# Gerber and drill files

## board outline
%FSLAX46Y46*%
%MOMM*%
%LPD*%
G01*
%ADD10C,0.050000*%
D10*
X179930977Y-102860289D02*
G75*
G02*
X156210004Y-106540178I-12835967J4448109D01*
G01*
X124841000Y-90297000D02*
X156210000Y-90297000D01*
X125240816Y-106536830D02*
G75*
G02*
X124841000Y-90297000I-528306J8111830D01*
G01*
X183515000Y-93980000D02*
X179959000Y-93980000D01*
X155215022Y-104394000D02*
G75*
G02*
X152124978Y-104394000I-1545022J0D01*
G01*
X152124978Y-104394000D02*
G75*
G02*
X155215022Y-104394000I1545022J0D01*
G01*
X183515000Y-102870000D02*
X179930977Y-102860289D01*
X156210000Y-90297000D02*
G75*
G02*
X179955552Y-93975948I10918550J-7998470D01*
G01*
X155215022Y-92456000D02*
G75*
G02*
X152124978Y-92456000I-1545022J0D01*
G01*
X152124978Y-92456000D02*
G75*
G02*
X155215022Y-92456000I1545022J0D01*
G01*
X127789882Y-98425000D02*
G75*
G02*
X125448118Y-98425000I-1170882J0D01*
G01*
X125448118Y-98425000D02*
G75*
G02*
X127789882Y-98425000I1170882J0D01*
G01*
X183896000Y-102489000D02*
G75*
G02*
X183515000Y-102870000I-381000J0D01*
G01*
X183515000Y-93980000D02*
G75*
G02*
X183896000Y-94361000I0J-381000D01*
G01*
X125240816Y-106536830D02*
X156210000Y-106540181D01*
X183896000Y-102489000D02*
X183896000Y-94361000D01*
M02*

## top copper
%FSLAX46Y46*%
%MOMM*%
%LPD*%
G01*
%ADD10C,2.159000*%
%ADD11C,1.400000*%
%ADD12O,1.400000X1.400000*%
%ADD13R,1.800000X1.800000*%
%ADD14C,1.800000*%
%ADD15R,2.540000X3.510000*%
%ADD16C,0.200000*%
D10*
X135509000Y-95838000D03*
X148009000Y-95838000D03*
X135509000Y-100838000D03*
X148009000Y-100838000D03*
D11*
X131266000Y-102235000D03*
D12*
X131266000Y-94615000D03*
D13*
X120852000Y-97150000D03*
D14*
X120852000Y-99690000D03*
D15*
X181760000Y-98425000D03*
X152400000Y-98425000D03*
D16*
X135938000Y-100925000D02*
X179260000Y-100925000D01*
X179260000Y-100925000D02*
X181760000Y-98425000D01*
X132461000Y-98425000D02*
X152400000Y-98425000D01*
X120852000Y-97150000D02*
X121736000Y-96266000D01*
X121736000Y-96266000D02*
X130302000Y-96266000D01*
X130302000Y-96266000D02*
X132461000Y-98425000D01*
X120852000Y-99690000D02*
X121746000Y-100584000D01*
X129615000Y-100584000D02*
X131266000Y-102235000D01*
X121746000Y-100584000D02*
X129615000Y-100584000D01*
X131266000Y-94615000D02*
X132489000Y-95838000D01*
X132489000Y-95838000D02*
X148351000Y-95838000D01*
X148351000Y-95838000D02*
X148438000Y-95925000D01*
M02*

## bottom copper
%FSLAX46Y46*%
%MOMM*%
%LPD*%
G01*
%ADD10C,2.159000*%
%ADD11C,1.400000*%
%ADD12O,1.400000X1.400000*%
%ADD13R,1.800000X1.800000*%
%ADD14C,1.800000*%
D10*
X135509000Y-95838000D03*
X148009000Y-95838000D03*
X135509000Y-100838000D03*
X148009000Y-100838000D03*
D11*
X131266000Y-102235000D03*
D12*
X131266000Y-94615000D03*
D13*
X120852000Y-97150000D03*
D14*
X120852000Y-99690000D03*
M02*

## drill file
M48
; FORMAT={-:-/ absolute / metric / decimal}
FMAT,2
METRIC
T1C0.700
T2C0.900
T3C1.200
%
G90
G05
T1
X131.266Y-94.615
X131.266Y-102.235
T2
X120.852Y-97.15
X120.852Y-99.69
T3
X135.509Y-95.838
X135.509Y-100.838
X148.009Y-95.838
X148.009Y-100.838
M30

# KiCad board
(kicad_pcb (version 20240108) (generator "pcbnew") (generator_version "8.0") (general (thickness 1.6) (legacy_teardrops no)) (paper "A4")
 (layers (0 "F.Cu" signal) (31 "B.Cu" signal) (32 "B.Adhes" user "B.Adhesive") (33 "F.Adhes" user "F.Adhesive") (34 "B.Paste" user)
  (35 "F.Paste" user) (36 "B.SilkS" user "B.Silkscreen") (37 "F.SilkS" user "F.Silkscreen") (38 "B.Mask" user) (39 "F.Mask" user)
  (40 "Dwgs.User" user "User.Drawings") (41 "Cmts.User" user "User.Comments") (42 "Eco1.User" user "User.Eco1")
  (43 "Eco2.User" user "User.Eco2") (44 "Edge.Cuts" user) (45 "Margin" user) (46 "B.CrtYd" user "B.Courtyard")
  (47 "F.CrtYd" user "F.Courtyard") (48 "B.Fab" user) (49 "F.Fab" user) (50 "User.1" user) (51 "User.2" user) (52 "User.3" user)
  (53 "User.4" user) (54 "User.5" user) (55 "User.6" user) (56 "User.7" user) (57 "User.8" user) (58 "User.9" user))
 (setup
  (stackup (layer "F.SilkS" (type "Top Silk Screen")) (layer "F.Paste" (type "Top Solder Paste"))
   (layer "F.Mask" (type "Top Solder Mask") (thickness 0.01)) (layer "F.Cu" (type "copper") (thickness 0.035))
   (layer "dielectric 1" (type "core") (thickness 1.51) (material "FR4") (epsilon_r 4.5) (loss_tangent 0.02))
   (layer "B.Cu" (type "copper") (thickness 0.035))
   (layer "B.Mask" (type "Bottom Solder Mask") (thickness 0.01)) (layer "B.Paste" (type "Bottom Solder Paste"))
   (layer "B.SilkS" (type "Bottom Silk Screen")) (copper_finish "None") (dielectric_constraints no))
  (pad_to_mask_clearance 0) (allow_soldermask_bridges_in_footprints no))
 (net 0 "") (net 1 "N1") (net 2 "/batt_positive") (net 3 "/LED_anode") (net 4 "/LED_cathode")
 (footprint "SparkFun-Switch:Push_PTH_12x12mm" (layer "F.Cu") (at 141.759 98.338)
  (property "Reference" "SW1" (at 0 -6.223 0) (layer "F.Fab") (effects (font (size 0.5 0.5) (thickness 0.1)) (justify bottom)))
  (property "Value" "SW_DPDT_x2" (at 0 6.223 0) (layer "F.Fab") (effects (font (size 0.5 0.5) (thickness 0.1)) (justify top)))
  (pad "1" thru_hole circle (at -6.25 -2.5) (size 2.159 2.159) (drill 1.2) (layers "*.Cu" "*.Mask") (remove_unused_layers no) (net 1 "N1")
   (solder_mask_margin 0.1016) (thermal_bridge_angle 0))
  (pad "1" thru_hole circle (at 6.25 -2.5) (size 2.159 2.159) (drill 1.2) (layers "*.Cu" "*.Mask") (remove_unused_layers no) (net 1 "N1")
   (solder_mask_margin 0.1016) (thermal_bridge_angle 0))
  (pad "2" thru_hole circle (at -6.25 2.5) (size 2.159 2.159) (drill 1.2) (layers "*.Cu" "*.Mask") (remove_unused_layers no)
   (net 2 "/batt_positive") (solder_mask_margin 0.1016) (thermal_bridge_angle 0))
  (pad "2" thru_hole circle (at 6.25 2.5) (size 2.159 2.159) (drill 1.2) (layers "*.Cu" "*.Mask") (remove_unused_layers no)
   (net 2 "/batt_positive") (solder_mask_margin 0.1016) (thermal_bridge_angle 0)))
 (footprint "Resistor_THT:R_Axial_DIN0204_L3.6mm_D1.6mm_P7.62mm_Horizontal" (layer "F.Cu") (at 131.266 102.235 90)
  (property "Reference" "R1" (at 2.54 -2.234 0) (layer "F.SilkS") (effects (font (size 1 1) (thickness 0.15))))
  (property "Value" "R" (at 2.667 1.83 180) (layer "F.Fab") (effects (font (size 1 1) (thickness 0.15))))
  (pad "1" thru_hole circle (at 0 0 90) (size 1.4 1.4) (drill 0.7) (layers "*.Cu" "*.Mask") (remove_unused_layers no) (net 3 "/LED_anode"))
  (pad "2" thru_hole oval (at 7.62 0 90) (size 1.4 1.4) (drill 0.7) (layers "*.Cu" "*.Mask") (remove_unused_layers no) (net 1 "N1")))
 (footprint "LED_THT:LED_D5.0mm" (layer "F.Cu") (at 120.852 97.15 -90)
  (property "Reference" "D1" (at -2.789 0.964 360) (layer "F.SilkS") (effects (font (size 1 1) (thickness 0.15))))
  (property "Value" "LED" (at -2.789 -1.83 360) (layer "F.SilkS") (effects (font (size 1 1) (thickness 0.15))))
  (pad "1" thru_hole rect (at 0 0 270) (size 1.8 1.8) (drill 0.9) (layers "*.Cu" "*.Mask") (remove_unused_layers no) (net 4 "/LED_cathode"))
  (pad "2" thru_hole circle (at 2.54 0 270) (size 1.8 1.8) (drill 0.9) (layers "*.Cu" "*.Mask") (remove_unused_layers no)
   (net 3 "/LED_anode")))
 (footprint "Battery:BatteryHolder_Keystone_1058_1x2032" (layer "F.Cu") (at 167.08 98.425 180)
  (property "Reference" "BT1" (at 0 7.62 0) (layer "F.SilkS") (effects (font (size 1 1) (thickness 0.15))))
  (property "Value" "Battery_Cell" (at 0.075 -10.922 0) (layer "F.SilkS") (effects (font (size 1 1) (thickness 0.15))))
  (pad "1" smd rect (at -14.68 0 180) (size 2.54 3.51) (layers "F.Cu" "F.Paste" "F.Mask") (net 2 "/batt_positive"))
  (pad "2" smd rect (at 14.68 0 180) (size 2.54 3.51) (layers "F.Cu" "F.Paste" "F.Mask") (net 4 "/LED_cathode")))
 (gr_arc (start 179.930977 102.860289) (mid 169.177546 111.836443) (end 156.21 106.540181) (stroke (width 0.05) (type default))
  (layer "Edge.Cuts"))
 (gr_line (start 124.841 90.297) (end 156.21 90.297) (stroke (width 0.05) (type default)) (layer "Edge.Cuts"))
 (gr_arc (start 125.240816 106.53683) (mid 116.585959 98.625071) (end 124.841 90.297001) (stroke (width 0.05) (type default))
  (layer "Edge.Cuts"))
 (gr_line (start 183.515 93.98) (end 179.959 93.98) (stroke (width 0.05) (type default)) (layer "Edge.Cuts"))
 (gr_circle (center 153.67 104.394) (end 153.924 105.918) (stroke (width 0.05) (type default)) (fill none) (layer "Edge.Cuts"))
 (gr_line (start 183.515 102.87) (end 179.930977 102.860289) (stroke (width 0.05) (type default)) (layer "Edge.Cuts"))
 (gr_arc (start 156.21 90.297) (mid 169.200795 84.920271) (end 179.955545 93.97595) (stroke (width 0.05) (type default)) (layer "Edge.Cuts"))
 (gr_circle (center 153.67 92.456) (end 153.924 93.98) (stroke (width 0.05) (type default)) (fill none) (layer "Edge.Cuts"))
 (gr_circle (center 126.619 98.425) (end 126.873 99.568) (stroke (width 0.05) (type default)) (fill none) (layer "Edge.Cuts"))
 (gr_arc (start 183.896 102.489) (mid 183.784408 102.758408) (end 183.515 102.87) (stroke (width 0.05) (type default)) (layer "Edge.Cuts"))
 (gr_arc (start 183.515 93.98) (mid 183.784408 94.091592) (end 183.896 94.361) (stroke (width 0.05) (type default)) (layer "Edge.Cuts"))
 (gr_line (start 125.240816 106.53683) (end 156.21 106.540181) (stroke (width 0.05) (type default)) (layer "Edge.Cuts"))
 (gr_line (start 183.896 102.489) (end 183.896 94.361) (stroke (width 0.05) (type default)) (layer "Edge.Cuts"))
 (segment (start 135.938 100.925) (end 179.26 100.925) (width 0.2) (layer "F.Cu") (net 2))
 (segment (start 179.26 100.925) (end 181.76 98.425) (width 0.2) (layer "F.Cu") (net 2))
 (segment (start 132.461 98.425) (end 152.4 98.425) (width 0.2) (layer "F.Cu") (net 4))
 (segment (start 120.852 97.15) (end 121.736 96.266) (width 0.2) (layer "F.Cu") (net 4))
 (segment (start 121.736 96.266) (end 130.302 96.266) (width 0.2) (layer "F.Cu") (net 4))
 (segment (start 130.302 96.266) (end 132.461 98.425) (width 0.2) (layer "F.Cu") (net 4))
 (segment (start 120.852 99.69) (end 121.746 100.584) (width 0.2) (layer "F.Cu") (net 3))
 (segment (start 129.615 100.584) (end 131.266 102.235) (width 0.2) (layer "F.Cu") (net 3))
 (segment (start 121.746 100.584) (end 129.615 100.584) (width 0.2) (layer "F.Cu") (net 3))
 (segment (start 131.266 94.615) (end 132.489 95.838) (width 0.2) (layer "F.Cu") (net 1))
 (segment (start 132.489 95.838) (end 148.351 95.838) (width 0.2) (layer "F.Cu") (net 1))
 (segment (start 148.351 95.838) (end 148.438 95.925) (width 0.2) (layer "F.Cu") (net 1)))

